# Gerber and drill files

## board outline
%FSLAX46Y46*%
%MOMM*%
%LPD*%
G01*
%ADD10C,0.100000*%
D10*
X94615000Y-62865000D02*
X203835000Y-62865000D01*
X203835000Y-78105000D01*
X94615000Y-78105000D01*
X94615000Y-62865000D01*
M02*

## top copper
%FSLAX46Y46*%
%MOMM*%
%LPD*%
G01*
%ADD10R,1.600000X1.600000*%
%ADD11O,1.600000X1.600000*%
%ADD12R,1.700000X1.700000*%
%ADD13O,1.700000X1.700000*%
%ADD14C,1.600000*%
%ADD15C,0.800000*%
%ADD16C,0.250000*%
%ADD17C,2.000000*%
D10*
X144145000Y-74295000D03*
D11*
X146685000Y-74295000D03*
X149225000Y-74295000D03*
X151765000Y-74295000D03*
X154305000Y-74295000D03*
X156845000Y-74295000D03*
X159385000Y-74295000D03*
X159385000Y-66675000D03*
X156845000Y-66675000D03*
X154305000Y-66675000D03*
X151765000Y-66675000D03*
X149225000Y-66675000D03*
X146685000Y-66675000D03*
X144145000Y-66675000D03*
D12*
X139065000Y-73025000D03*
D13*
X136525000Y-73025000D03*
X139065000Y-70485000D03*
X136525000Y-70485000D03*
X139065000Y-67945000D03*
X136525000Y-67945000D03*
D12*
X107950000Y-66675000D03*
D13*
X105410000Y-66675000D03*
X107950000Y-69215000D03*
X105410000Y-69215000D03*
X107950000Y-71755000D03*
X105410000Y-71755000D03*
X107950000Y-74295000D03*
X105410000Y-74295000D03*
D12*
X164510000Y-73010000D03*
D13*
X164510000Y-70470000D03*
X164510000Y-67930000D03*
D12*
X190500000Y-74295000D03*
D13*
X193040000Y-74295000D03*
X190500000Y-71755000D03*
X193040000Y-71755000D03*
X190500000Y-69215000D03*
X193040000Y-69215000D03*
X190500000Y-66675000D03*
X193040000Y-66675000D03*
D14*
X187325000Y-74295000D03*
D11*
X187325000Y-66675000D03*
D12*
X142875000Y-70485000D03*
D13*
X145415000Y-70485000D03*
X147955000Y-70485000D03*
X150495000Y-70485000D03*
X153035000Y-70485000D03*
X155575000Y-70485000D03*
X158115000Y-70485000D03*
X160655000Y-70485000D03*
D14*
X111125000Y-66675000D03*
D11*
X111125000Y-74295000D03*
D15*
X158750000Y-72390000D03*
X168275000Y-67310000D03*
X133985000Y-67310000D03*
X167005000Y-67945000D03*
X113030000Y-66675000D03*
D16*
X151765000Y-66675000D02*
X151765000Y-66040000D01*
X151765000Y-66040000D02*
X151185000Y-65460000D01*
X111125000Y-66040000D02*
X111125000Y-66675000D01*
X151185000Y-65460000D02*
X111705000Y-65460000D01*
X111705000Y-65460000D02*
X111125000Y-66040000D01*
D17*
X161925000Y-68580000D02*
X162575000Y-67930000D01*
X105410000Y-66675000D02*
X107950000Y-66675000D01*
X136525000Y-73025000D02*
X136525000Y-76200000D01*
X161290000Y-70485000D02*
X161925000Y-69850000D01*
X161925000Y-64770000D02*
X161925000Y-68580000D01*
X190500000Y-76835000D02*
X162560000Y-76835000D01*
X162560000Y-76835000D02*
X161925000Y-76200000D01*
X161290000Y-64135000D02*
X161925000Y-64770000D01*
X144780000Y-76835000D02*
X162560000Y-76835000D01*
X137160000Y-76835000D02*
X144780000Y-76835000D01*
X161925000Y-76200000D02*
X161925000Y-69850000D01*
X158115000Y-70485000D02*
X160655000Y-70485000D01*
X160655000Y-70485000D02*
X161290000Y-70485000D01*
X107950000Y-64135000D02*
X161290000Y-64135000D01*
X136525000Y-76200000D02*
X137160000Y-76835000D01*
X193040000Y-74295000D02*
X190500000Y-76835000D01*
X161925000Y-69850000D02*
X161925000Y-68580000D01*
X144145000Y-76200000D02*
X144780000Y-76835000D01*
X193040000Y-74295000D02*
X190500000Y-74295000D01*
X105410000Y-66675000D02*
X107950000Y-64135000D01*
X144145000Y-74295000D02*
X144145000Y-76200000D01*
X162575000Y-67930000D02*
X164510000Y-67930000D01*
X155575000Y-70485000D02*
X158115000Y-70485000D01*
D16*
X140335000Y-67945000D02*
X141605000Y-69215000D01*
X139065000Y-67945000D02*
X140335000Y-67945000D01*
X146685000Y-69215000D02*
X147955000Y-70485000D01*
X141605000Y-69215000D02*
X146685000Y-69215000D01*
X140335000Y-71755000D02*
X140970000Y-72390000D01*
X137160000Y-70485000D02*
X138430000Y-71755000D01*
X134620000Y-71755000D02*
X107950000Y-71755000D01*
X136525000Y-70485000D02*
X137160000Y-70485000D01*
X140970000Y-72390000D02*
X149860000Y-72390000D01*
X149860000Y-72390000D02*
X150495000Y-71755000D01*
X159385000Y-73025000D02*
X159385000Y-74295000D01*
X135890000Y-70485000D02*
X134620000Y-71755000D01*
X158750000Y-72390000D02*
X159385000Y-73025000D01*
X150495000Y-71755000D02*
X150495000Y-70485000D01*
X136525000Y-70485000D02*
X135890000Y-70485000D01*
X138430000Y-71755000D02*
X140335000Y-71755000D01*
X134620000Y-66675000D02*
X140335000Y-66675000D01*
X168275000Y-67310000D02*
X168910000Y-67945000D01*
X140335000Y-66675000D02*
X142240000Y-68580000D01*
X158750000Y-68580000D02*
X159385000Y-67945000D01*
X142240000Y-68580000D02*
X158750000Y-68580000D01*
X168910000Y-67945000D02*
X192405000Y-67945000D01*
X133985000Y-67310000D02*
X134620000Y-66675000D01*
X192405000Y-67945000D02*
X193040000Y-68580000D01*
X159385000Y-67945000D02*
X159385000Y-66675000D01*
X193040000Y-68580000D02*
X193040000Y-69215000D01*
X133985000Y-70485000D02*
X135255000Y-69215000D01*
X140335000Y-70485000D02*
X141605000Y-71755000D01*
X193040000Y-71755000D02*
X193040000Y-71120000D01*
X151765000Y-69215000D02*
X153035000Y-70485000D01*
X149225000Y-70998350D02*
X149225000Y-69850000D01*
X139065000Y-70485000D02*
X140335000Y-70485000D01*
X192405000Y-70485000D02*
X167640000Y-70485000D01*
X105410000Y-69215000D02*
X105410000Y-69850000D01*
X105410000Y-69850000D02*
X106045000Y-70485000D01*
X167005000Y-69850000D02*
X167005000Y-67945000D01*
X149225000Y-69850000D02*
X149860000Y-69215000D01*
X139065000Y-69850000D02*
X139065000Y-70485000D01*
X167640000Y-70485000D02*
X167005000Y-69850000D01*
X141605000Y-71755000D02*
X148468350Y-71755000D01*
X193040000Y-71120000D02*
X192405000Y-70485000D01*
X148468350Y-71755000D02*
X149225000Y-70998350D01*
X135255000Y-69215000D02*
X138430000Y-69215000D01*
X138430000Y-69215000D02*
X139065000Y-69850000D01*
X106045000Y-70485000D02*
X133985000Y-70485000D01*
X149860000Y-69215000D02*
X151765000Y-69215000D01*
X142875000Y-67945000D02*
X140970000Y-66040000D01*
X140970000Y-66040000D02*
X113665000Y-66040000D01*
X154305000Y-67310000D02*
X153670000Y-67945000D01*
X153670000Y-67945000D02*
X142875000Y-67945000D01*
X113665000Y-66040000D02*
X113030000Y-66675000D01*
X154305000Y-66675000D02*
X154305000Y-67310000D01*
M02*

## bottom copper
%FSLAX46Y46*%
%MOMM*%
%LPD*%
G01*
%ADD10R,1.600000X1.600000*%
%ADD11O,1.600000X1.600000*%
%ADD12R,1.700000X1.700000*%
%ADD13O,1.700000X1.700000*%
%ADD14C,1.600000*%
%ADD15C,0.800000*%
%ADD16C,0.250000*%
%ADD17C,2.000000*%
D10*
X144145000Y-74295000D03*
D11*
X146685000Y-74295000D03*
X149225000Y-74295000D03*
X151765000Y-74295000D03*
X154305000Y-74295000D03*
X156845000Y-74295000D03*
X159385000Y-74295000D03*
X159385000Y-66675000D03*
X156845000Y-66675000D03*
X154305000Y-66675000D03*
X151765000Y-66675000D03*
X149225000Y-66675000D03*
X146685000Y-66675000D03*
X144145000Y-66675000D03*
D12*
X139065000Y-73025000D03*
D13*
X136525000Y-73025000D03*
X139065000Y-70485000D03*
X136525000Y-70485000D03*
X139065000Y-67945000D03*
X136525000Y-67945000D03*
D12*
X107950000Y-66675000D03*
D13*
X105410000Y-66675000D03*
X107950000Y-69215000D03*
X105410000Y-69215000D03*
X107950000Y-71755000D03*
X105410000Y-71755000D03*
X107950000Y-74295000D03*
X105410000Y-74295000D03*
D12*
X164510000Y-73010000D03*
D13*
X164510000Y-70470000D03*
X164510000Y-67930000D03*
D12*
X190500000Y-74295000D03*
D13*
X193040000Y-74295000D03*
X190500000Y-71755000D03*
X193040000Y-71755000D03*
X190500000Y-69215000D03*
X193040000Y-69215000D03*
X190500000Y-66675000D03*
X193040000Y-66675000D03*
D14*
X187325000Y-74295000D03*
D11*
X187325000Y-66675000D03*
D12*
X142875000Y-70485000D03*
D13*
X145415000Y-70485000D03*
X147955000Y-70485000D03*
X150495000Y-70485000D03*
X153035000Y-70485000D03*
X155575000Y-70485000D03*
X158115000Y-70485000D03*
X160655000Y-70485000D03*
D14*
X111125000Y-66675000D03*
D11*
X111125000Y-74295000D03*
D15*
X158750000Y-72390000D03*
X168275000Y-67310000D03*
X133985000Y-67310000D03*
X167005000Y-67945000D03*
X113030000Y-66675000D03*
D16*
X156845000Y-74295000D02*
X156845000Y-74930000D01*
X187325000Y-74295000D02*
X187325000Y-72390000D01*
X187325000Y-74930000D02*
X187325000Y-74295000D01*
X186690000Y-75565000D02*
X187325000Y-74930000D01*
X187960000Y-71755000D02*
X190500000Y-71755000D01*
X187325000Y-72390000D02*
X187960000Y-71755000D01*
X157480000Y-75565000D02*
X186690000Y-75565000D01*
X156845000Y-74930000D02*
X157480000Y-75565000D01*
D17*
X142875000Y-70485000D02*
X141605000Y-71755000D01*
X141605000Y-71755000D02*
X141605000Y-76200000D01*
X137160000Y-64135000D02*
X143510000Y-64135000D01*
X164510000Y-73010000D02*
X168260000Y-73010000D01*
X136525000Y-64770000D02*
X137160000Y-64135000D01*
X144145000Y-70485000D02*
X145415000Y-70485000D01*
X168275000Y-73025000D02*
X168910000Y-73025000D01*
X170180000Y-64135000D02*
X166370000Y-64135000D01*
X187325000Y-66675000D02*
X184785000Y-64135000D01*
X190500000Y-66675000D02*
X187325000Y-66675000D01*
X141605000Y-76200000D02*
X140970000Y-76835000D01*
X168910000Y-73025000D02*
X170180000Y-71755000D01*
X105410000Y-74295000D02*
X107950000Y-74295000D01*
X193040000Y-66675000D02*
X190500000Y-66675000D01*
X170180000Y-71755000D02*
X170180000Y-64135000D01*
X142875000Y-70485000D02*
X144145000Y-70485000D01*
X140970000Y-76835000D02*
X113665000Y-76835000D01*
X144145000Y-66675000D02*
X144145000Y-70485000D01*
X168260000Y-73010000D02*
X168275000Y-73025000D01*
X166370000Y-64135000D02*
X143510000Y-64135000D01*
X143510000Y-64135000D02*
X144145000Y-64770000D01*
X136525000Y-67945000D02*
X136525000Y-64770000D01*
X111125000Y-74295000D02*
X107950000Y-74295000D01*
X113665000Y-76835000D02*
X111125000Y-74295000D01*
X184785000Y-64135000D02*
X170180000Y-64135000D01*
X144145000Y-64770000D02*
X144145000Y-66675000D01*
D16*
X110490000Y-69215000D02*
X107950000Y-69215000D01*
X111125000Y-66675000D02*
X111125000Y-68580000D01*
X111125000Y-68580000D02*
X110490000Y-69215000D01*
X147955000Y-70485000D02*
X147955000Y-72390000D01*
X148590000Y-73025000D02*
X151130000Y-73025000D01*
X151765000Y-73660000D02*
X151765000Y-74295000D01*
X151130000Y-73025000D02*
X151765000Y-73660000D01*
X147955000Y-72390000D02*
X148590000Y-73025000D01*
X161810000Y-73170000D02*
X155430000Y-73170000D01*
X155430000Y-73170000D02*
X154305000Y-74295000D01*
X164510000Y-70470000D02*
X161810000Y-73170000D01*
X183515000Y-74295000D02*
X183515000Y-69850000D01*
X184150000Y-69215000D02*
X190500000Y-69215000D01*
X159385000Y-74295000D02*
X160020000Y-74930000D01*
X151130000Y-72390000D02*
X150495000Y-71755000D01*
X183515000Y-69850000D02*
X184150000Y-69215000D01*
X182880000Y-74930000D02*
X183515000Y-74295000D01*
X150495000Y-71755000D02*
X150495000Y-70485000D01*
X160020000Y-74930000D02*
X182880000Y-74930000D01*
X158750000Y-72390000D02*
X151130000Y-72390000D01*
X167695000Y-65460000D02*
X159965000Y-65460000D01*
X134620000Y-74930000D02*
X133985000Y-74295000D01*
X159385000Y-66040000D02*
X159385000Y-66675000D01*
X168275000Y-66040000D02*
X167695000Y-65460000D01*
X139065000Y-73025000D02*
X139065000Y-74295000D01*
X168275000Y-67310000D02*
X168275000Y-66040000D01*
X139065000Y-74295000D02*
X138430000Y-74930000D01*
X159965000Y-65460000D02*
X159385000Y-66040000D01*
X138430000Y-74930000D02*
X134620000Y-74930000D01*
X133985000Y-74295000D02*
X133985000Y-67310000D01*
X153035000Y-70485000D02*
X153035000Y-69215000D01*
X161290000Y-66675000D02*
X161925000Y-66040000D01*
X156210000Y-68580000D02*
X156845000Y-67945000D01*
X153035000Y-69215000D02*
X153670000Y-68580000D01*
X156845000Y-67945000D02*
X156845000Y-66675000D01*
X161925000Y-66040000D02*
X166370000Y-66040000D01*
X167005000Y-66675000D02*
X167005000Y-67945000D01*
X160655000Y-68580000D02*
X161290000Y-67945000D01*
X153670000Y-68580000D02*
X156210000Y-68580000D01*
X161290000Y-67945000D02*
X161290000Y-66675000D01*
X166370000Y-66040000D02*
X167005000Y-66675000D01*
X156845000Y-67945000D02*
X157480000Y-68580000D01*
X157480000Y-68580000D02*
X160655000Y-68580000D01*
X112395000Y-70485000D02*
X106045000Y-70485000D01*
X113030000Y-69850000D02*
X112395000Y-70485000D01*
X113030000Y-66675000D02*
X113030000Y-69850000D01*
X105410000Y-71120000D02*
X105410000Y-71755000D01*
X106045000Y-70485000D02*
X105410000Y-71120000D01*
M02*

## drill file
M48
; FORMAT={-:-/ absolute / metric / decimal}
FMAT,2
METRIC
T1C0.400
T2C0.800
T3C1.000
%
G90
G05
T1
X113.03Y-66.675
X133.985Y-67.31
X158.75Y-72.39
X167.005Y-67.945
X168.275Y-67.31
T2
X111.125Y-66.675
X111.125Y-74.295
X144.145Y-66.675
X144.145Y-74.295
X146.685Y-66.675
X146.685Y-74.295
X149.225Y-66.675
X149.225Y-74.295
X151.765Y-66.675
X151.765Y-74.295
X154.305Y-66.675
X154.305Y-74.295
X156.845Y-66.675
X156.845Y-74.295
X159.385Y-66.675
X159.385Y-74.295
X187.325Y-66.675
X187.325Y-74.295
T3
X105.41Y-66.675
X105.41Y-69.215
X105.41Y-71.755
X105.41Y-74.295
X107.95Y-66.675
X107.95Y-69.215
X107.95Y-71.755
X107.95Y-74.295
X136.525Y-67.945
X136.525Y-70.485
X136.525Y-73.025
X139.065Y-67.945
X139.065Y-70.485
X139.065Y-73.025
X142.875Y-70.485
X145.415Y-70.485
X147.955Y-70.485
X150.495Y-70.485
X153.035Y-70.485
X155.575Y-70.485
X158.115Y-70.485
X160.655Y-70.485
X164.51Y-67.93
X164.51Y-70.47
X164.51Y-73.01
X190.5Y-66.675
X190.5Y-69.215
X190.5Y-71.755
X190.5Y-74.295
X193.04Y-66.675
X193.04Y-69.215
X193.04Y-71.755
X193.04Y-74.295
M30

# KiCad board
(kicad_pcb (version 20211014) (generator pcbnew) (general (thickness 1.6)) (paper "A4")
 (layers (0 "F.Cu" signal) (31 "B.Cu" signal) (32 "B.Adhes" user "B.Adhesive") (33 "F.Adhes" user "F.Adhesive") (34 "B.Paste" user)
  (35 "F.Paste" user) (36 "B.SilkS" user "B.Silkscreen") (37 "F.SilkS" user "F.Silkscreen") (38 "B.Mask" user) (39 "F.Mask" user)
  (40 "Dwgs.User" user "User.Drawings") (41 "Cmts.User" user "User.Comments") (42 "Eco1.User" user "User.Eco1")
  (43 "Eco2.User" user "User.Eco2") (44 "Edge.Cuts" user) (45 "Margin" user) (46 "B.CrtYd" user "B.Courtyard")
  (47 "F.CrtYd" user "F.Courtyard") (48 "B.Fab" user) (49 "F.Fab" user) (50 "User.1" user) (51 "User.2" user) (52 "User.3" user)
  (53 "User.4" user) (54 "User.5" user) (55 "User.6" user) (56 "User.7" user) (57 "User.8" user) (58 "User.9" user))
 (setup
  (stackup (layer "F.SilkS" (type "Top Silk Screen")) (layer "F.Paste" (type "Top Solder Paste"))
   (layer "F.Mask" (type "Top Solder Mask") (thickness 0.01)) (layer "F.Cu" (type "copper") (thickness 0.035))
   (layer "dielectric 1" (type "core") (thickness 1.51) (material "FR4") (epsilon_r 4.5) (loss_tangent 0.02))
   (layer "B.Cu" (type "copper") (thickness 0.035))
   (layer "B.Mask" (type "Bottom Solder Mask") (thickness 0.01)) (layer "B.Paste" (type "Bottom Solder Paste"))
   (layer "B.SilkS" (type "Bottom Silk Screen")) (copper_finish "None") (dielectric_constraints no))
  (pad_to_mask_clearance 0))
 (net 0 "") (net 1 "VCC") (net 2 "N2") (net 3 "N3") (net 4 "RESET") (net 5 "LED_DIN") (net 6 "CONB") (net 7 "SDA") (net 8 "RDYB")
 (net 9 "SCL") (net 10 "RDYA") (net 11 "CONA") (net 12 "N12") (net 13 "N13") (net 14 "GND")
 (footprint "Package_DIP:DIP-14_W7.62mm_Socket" (layer "F.Cu") (at 144.145 74.295 90)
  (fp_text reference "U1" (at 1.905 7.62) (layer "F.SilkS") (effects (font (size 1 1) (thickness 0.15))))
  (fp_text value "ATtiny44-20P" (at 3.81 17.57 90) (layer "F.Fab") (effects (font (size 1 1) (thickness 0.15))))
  (pad "1" thru_hole rect (at 0 0 90) (size 1.6 1.6) (drill 0.8) (layers *.Cu *.Mask) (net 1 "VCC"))
  (pad "2" thru_hole oval (at 0 2.54 90) (size 1.6 1.6) (drill 0.8) (layers *.Cu *.Mask) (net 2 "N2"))
  (pad "3" thru_hole oval (at 0 5.08 90) (size 1.6 1.6) (drill 0.8) (layers *.Cu *.Mask) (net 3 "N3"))
  (pad "4" thru_hole oval (at 0 7.62 90) (size 1.6 1.6) (drill 0.8) (layers *.Cu *.Mask) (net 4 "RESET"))
  (pad "5" thru_hole oval (at 0 10.16 90) (size 1.6 1.6) (drill 0.8) (layers *.Cu *.Mask) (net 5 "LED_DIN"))
  (pad "6" thru_hole oval (at 0 12.7 90) (size 1.6 1.6) (drill 0.8) (layers *.Cu *.Mask) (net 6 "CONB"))
  (pad "7" thru_hole oval (at 0 15.24 90) (size 1.6 1.6) (drill 0.8) (layers *.Cu *.Mask) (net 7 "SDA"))
  (pad "8" thru_hole oval (at 7.62 15.24 90) (size 1.6 1.6) (drill 0.8) (layers *.Cu *.Mask) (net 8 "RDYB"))
  (pad "9" thru_hole oval (at 7.62 12.7 90) (size 1.6 1.6) (drill 0.8) (layers *.Cu *.Mask) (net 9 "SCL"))
  (pad "10" thru_hole oval (at 7.62 10.16 90) (size 1.6 1.6) (drill 0.8) (layers *.Cu *.Mask) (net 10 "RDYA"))
  (pad "11" thru_hole oval (at 7.62 7.62 90) (size 1.6 1.6) (drill 0.8) (layers *.Cu *.Mask) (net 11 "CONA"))
  (pad "12" thru_hole oval (at 7.62 5.08 90) (size 1.6 1.6) (drill 0.8) (layers *.Cu *.Mask) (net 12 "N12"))
  (pad "13" thru_hole oval (at 7.62 2.54 90) (size 1.6 1.6) (drill 0.8) (layers *.Cu *.Mask) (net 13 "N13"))
  (pad "14" thru_hole oval (at 7.62 0 90) (size 1.6 1.6) (drill 0.8) (layers *.Cu *.Mask) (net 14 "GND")))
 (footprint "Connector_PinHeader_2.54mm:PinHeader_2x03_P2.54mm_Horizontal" (layer "F.Cu") (at 139.065 73.025 180)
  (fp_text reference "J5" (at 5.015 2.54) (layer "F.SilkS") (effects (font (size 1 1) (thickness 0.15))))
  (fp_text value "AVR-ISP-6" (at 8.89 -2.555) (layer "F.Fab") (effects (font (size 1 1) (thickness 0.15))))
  (pad "1" thru_hole rect (at 0 0 180) (size 1.7 1.7) (drill 1) (layers *.Cu *.Mask) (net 8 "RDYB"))
  (pad "2" thru_hole oval (at 2.54 0 180) (size 1.7 1.7) (drill 1) (layers *.Cu *.Mask) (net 1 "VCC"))
  (pad "3" thru_hole oval (at 0 2.54 180) (size 1.7 1.7) (drill 1) (layers *.Cu *.Mask) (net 9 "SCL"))
  (pad "4" thru_hole oval (at 2.54 2.54 180) (size 1.7 1.7) (drill 1) (layers *.Cu *.Mask) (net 7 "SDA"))
  (pad "5" thru_hole oval (at 0 5.08 180) (size 1.7 1.7) (drill 1) (layers *.Cu *.Mask) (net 4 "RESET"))
  (pad "6" thru_hole oval (at 2.54 5.08 180) (size 1.7 1.7) (drill 1) (layers *.Cu *.Mask) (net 14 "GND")))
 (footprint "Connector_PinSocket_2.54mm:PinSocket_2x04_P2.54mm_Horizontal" (layer "F.Cu") (at 107.95 66.675)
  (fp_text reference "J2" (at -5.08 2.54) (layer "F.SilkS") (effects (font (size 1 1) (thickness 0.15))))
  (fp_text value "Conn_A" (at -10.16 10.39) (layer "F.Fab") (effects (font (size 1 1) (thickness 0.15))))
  (pad "1" thru_hole rect (at 0 0) (size 1.7 1.7) (drill 1) (layers *.Cu *.Mask) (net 1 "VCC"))
  (pad "2" thru_hole oval (at -2.54 0) (size 1.7 1.7) (drill 1) (layers *.Cu *.Mask) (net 1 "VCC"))
  (pad "3" thru_hole oval (at 0 2.54) (size 1.7 1.7) (drill 1) (layers *.Cu *.Mask) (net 11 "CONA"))
  (pad "4" thru_hole oval (at -2.54 2.54) (size 1.7 1.7) (drill 1) (layers *.Cu *.Mask) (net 9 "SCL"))
  (pad "5" thru_hole oval (at 0 5.08) (size 1.7 1.7) (drill 1) (layers *.Cu *.Mask) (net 7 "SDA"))
  (pad "6" thru_hole oval (at -2.54 5.08) (size 1.7 1.7) (drill 1) (layers *.Cu *.Mask) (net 10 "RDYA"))
  (pad "7" thru_hole oval (at 0 7.62) (size 1.7 1.7) (drill 1) (layers *.Cu *.Mask) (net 14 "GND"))
  (pad "8" thru_hole oval (at -2.54 7.62) (size 1.7 1.7) (drill 1) (layers *.Cu *.Mask) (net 14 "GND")))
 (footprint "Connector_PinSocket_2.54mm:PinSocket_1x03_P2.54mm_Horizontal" (layer "F.Cu") (at 164.51 73.01 180)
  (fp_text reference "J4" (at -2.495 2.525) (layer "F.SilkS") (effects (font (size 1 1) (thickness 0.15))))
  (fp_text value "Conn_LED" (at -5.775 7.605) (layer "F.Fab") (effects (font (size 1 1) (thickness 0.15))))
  (pad "1" thru_hole rect (at 0 0 180) (size 1.7 1.7) (drill 1) (layers *.Cu *.Mask) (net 14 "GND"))
  (pad "2" thru_hole oval (at 0 2.54 180) (size 1.7 1.7) (drill 1) (layers *.Cu *.Mask) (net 5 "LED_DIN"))
  (pad "3" thru_hole oval (at 0 5.08 180) (size 1.7 1.7) (drill 1) (layers *.Cu *.Mask) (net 1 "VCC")))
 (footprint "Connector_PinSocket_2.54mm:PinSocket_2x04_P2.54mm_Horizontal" (layer "F.Cu") (at 190.5 74.295 180)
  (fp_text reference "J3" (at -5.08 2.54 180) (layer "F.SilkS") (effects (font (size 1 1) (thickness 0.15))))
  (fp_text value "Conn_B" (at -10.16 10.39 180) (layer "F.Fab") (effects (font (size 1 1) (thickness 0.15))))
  (pad "1" thru_hole rect (at 0 0 180) (size 1.7 1.7) (drill 1) (layers *.Cu *.Mask) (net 1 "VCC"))
  (pad "2" thru_hole oval (at -2.54 0 180) (size 1.7 1.7) (drill 1) (layers *.Cu *.Mask) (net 1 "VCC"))
  (pad "3" thru_hole oval (at 0 2.54 180) (size 1.7 1.7) (drill 1) (layers *.Cu *.Mask) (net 6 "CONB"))
  (pad "4" thru_hole oval (at -2.54 2.54 180) (size 1.7 1.7) (drill 1) (layers *.Cu *.Mask) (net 9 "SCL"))
  (pad "5" thru_hole oval (at 0 5.08 180) (size 1.7 1.7) (drill 1) (layers *.Cu *.Mask) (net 7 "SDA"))
  (pad "6" thru_hole oval (at -2.54 5.08 180) (size 1.7 1.7) (drill 1) (layers *.Cu *.Mask) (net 8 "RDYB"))
  (pad "7" thru_hole oval (at 0 7.62 180) (size 1.7 1.7) (drill 1) (layers *.Cu *.Mask) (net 14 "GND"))
  (pad "8" thru_hole oval (at -2.54 7.62 180) (size 1.7 1.7) (drill 1) (layers *.Cu *.Mask) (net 14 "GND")))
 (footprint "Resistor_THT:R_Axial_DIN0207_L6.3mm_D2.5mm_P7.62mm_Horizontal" (layer "B.Cu") (at 187.325 74.295 90)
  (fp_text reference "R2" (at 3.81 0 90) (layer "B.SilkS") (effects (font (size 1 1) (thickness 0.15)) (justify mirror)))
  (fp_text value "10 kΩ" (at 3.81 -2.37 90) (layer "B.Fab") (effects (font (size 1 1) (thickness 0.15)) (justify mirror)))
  (pad "1" thru_hole circle (at 0 0 90) (size 1.6 1.6) (drill 0.8) (layers *.Cu *.Mask) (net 6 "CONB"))
  (pad "2" thru_hole oval (at 7.62 0 90) (size 1.6 1.6) (drill 0.8) (layers *.Cu *.Mask) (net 14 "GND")))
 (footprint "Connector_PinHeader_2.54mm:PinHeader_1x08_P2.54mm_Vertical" (layer "B.Cu") (at 142.875 70.485 -90)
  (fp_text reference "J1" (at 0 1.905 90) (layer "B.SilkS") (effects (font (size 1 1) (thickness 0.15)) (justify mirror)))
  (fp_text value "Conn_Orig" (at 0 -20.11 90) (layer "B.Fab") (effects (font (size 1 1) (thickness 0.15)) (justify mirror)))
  (pad "1" thru_hole rect (at 0 0 270) (size 1.7 1.7) (drill 1) (layers *.Cu *.Mask) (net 14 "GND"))
  (pad "2" thru_hole oval (at 0 -2.54 270) (size 1.7 1.7) (drill 1) (layers *.Cu *.Mask) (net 14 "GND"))
  (pad "3" thru_hole oval (at 0 -5.08 270) (size 1.7 1.7) (drill 1) (layers *.Cu *.Mask) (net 4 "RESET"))
  (pad "4" thru_hole oval (at 0 -7.62 270) (size 1.7 1.7) (drill 1) (layers *.Cu *.Mask) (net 7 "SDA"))
  (pad "5" thru_hole oval (at 0 -10.16 270) (size 1.7 1.7) (drill 1) (layers *.Cu *.Mask) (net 9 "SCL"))
  (pad "6" thru_hole oval (at 0 -12.7 270) (size 1.7 1.7) (drill 1) (layers *.Cu *.Mask) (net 1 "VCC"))
  (pad "7" thru_hole oval (at 0 -15.24 270) (size 1.7 1.7) (drill 1) (layers *.Cu *.Mask) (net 1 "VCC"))
  (pad "8" thru_hole oval (at 0 -17.78 270) (size 1.7 1.7) (drill 1) (layers *.Cu *.Mask) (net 1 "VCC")))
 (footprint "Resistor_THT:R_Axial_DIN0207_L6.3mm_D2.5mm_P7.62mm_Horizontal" (layer "B.Cu") (at 111.125 66.675 -90)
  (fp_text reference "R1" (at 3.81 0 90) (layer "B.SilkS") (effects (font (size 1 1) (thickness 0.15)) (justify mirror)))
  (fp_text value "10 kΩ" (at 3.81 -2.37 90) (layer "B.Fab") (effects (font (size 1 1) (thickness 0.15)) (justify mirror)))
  (pad "1" thru_hole circle (at 0 0 270) (size 1.6 1.6) (drill 0.8) (layers *.Cu *.Mask) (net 11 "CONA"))
  (pad "2" thru_hole oval (at 7.62 0 270) (size 1.6 1.6) (drill 0.8) (layers *.Cu *.Mask) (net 14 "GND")))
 (gr_rect (start 94.615 62.865) (end 203.835 78.105) (layer "Edge.Cuts") (width 0.1) (fill none))
 (segment (start 156.845 74.295) (end 156.845 74.93) (width 0.25) (layer "B.Cu") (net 6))
 (segment (start 187.325 74.295) (end 187.325 72.39) (width 0.25) (layer "B.Cu") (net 6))
 (segment (start 187.325 74.93) (end 187.325 74.295) (width 0.25) (layer "B.Cu") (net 6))
 (segment (start 186.69 75.565) (end 187.325 74.93) (width 0.25) (layer "B.Cu") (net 6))
 (segment (start 187.96 71.755) (end 190.5 71.755) (width 0.25) (layer "B.Cu") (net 6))
 (segment (start 187.325 72.39) (end 187.96 71.755) (width 0.25) (layer "B.Cu") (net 6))
 (segment (start 157.48 75.565) (end 186.69 75.565) (width 0.25) (layer "B.Cu") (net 6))
 (segment (start 156.845 74.93) (end 157.48 75.565) (width 0.25) (layer "B.Cu") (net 6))
 (segment (start 142.875 70.485) (end 141.605 71.755) (width 2) (layer "B.Cu") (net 14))
 (segment (start 141.605 71.755) (end 141.605 76.2) (width 2) (layer "B.Cu") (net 14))
 (segment (start 137.16 64.135) (end 143.51 64.135) (width 2) (layer "B.Cu") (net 14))
 (segment (start 164.51 73.01) (end 168.26 73.01) (width 2) (layer "B.Cu") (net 14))
 (segment (start 136.525 64.77) (end 137.16 64.135) (width 2) (layer "B.Cu") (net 14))
 (segment (start 144.145 70.485) (end 145.415 70.485) (width 2) (layer "B.Cu") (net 14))
 (segment (start 168.275 73.025) (end 168.91 73.025) (width 2) (layer "B.Cu") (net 14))
 (segment (start 170.18 64.135) (end 166.37 64.135) (width 2) (layer "B.Cu") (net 14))
 (segment (start 187.325 66.675) (end 184.785 64.135) (width 2) (layer "B.Cu") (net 14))
 (segment (start 190.5 66.675) (end 187.325 66.675) (width 2) (layer "B.Cu") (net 14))
 (segment (start 141.605 76.2) (end 140.97 76.835) (width 2) (layer "B.Cu") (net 14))
 (segment (start 168.91 73.025) (end 170.18 71.755) (width 2) (layer "B.Cu") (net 14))
 (segment (start 105.41 74.295) (end 107.95 74.295) (width 2) (layer "B.Cu") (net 14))
 (segment (start 193.04 66.675) (end 190.5 66.675) (width 2) (layer "B.Cu") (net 14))
 (segment (start 170.18 71.755) (end 170.18 64.135) (width 2) (layer "B.Cu") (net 14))
 (segment (start 142.875 70.485) (end 144.145 70.485) (width 2) (layer "B.Cu") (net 14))
 (segment (start 140.97 76.835) (end 113.665 76.835) (width 2) (layer "B.Cu") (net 14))
 (segment (start 144.145 66.675) (end 144.145 70.485) (width 2) (layer "B.Cu") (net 14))
 (segment (start 168.26 73.01) (end 168.275 73.025) (width 2) (layer "B.Cu") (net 14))
 (segment (start 166.37 64.135) (end 143.51 64.135) (width 2) (layer "B.Cu") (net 14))
 (segment (start 143.51 64.135) (end 144.145 64.77) (width 2) (layer "B.Cu") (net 14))
 (segment (start 136.525 67.945) (end 136.525 64.77) (width 2) (layer "B.Cu") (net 14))
 (segment (start 111.125 74.295) (end 107.95 74.295) (width 2) (layer "B.Cu") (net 14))
 (segment (start 113.665 76.835) (end 111.125 74.295) (width 2) (layer "B.Cu") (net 14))
 (segment (start 184.785 64.135) (end 170.18 64.135) (width 2) (layer "B.Cu") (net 14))
 (segment (start 144.145 64.77) (end 144.145 66.675) (width 2) (layer "B.Cu") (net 14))
 (segment (start 151.765 66.675) (end 151.765 66.04) (width 0.25) (layer "F.Cu") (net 11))
 (segment (start 151.765 66.04) (end 151.185 65.46) (width 0.25) (layer "F.Cu") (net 11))
 (segment (start 111.125 66.04) (end 111.125 66.675) (width 0.25) (layer "F.Cu") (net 11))
 (segment (start 151.185 65.46) (end 111.705 65.46) (width 0.25) (layer "F.Cu") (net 11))
 (segment (start 111.705 65.46) (end 111.125 66.04) (width 0.25) (layer "F.Cu") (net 11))
 (segment (start 110.49 69.215) (end 107.95 69.215) (width 0.25) (layer "B.Cu") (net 11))
 (segment (start 111.125 66.675) (end 111.125 68.58) (width 0.25) (layer "B.Cu") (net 11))
 (segment (start 111.125 68.58) (end 110.49 69.215) (width 0.25) (layer "B.Cu") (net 11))
 (segment (start 161.925 68.58) (end 162.575 67.93) (width 2) (layer "F.Cu") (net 1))
 (segment (start 105.41 66.675) (end 107.95 66.675) (width 2) (layer "F.Cu") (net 1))
 (segment (start 136.525 73.025) (end 136.525 76.2) (width 2) (layer "F.Cu") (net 1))
 (segment (start 161.29 70.485) (end 161.925 69.85) (width 2) (layer "F.Cu") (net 1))
 (segment (start 161.925 64.77) (end 161.925 68.58) (width 2) (layer "F.Cu") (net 1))
 (segment (start 190.5 76.835) (end 162.56 76.835) (width 2) (layer "F.Cu") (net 1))
 (segment (start 162.56 76.835) (end 161.925 76.2) (width 2) (layer "F.Cu") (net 1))
 (segment (start 161.29 64.135) (end 161.925 64.77) (width 2) (layer "F.Cu") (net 1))
 (segment (start 144.78 76.835) (end 162.56 76.835) (width 2) (layer "F.Cu") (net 1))
 (segment (start 137.16 76.835) (end 144.78 76.835) (width 2) (layer "F.Cu") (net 1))
 (segment (start 161.925 76.2) (end 161.925 69.85) (width 2) (layer "F.Cu") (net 1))
 (segment (start 158.115 70.485) (end 160.655 70.485) (width 2) (layer "F.Cu") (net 1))
 (segment (start 160.655 70.485) (end 161.29 70.485) (width 2) (layer "F.Cu") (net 1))
 (segment (start 107.95 64.135) (end 161.29 64.135) (width 2) (layer "F.Cu") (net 1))
 (segment (start 136.525 76.2) (end 137.16 76.835) (width 2) (layer "F.Cu") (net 1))
 (segment (start 193.04 74.295) (end 190.5 76.835) (width 2) (layer "F.Cu") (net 1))
 (segment (start 161.925 69.85) (end 161.925 68.58) (width 2) (layer "F.Cu") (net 1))
 (segment (start 144.145 76.2) (end 144.78 76.835) (width 2) (layer "F.Cu") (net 1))
 (segment (start 193.04 74.295) (end 190.5 74.295) (width 2) (layer "F.Cu") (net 1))
 (segment (start 105.41 66.675) (end 107.95 64.135) (width 2) (layer "F.Cu") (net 1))
 (segment (start 144.145 74.295) (end 144.145 76.2) (width 2) (layer "F.Cu") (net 1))
 (segment (start 162.575 67.93) (end 164.51 67.93) (width 2) (layer "F.Cu") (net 1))
 (segment (start 155.575 70.485) (end 158.115 70.485) (width 2) (layer "F.Cu") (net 1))
 (segment (start 140.335 67.945) (end 141.605 69.215) (width 0.25) (layer "F.Cu") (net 4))
 (segment (start 139.065 67.945) (end 140.335 67.945) (width 0.25) (layer "F.Cu") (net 4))
 (segment (start 146.685 69.215) (end 147.955 70.485) (width 0.25) (layer "F.Cu") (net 4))
 (segment (start 141.605 69.215) (end 146.685 69.215) (width 0.25) (layer "F.Cu") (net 4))
 (segment (start 147.955 70.485) (end 147.955 72.39) (width 0.25) (layer "B.Cu") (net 4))
 (segment (start 148.59 73.025) (end 151.13 73.025) (width 0.25) (layer "B.Cu") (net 4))
 (segment (start 151.765 73.66) (end 151.765 74.295) (width 0.25) (layer "B.Cu") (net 4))
 (segment (start 151.13 73.025) (end 151.765 73.66) (width 0.25) (layer "B.Cu") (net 4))
 (segment (start 147.955 72.39) (end 148.59 73.025) (width 0.25) (layer "B.Cu") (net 4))
 (segment (start 161.81 73.17) (end 155.43 73.17) (width 0.25) (layer "B.Cu") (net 5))
 (segment (start 155.43 73.17) (end 154.305 74.295) (width 0.25) (layer "B.Cu") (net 5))
 (segment (start 164.51 70.47) (end 161.81 73.17) (width 0.25) (layer "B.Cu") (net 5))
 (segment (start 140.335 71.755) (end 140.97 72.39) (width 0.25) (layer "F.Cu") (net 7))
 (segment (start 137.16 70.485) (end 138.43 71.755) (width 0.25) (layer "F.Cu") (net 7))
 (segment (start 134.62 71.755) (end 107.95 71.755) (width 0.25) (layer "F.Cu") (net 7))
 (segment (start 136.525 70.485) (end 137.16 70.485) (width 0.25) (layer "F.Cu") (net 7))
 (segment (start 140.97 72.39) (end 149.86 72.39) (width 0.25) (layer "F.Cu") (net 7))
 (segment (start 149.86 72.39) (end 150.495 71.755) (width 0.25) (layer "F.Cu") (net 7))
 (segment (start 159.385 73.025) (end 159.385 74.295) (width 0.25) (layer "F.Cu") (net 7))
 (segment (start 135.89 70.485) (end 134.62 71.755) (width 0.25) (layer "F.Cu") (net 7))
 (segment (start 158.75 72.39) (end 159.385 73.025) (width 0.25) (layer "F.Cu") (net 7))
 (segment (start 150.495 71.755) (end 150.495 70.485) (width 0.25) (layer "F.Cu") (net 7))
 (segment (start 136.525 70.485) (end 135.89 70.485) (width 0.25) (layer "F.Cu") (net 7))
 (segment (start 138.43 71.755) (end 140.335 71.755) (width 0.25) (layer "F.Cu") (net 7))
 (via (at 158.75 72.39) (size 0.8) (drill 0.4) (layers "F.Cu" "B.Cu") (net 7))
 (segment (start 183.515 74.295) (end 183.515 69.85) (width 0.25) (layer "B.Cu") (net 7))
 (segment (start 184.15 69.215) (end 190.5 69.215) (width 0.25) (layer "B.Cu") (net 7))
 (segment (start 159.385 74.295) (end 160.02 74.93) (width 0.25) (layer "B.Cu") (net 7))
 (segment (start 151.13 72.39) (end 150.495 71.755) (width 0.25) (layer "B.Cu") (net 7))
 (segment (start 183.515 69.85) (end 184.15 69.215) (width 0.25) (layer "B.Cu") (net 7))
 (segment (start 182.88 74.93) (end 183.515 74.295) (width 0.25) (layer "B.Cu") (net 7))
 (segment (start 150.495 71.755) (end 150.495 70.485) (width 0.25) (layer "B.Cu") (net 7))
 (segment (start 160.02 74.93) (end 182.88 74.93) (width 0.25) (layer "B.Cu") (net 7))
 (segment (start 158.75 72.39) (end 151.13 72.39) (width 0.25) (layer "B.Cu") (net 7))
 (segment (start 134.62 66.675) (end 140.335 66.675) (width 0.25) (layer "F.Cu") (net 8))
 (segment (start 168.275 67.31) (end 168.91 67.945) (width 0.25) (layer "F.Cu") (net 8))
 (segment (start 140.335 66.675) (end 142.24 68.58) (width 0.25) (layer "F.Cu") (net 8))
 (segment (start 158.75 68.58) (end 159.385 67.945) (width 0.25) (layer "F.Cu") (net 8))
 (segment (start 142.24 68.58) (end 158.75 68.58) (width 0.25) (layer "F.Cu") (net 8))
 (segment (start 168.91 67.945) (end 192.405 67.945) (width 0.25) (layer "F.Cu") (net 8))
 (segment (start 133.985 67.31) (end 134.62 66.675) (width 0.25) (layer "F.Cu") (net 8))
 (segment (start 192.405 67.945) (end 193.04 68.58) (width 0.25) (layer "F.Cu") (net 8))
 (segment (start 159.385 67.945) (end 159.385 66.675) (width 0.25) (layer "F.Cu") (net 8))
 (segment (start 193.04 68.58) (end 193.04 69.215) (width 0.25) (layer "F.Cu") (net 8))
 (via (at 168.275 67.31) (size 0.8) (drill 0.4) (layers "F.Cu" "B.Cu") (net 8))
 (via (at 133.985 67.31) (size 0.8) (drill 0.4) (layers "F.Cu" "B.Cu") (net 8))
 (segment (start 167.695 65.46) (end 159.965 65.46) (width 0.25) (layer "B.Cu") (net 8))
 (segment (start 134.62 74.93) (end 133.985 74.295) (width 0.25) (layer "B.Cu") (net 8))
 (segment (start 159.385 66.04) (end 159.385 66.675) (width 0.25) (layer "B.Cu") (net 8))
 (segment (start 168.275 66.04) (end 167.695 65.46) (width 0.25) (layer "B.Cu") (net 8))
 (segment (start 139.065 73.025) (end 139.065 74.295) (width 0.25) (layer "B.Cu") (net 8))
 (segment (start 168.275 67.31) (end 168.275 66.04) (width 0.25) (layer "B.Cu") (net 8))
 (segment (start 139.065 74.295) (end 138.43 74.93) (width 0.25) (layer "B.Cu") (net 8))
 (segment (start 159.965 65.46) (end 159.385 66.04) (width 0.25) (layer "B.Cu") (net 8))
 (segment (start 138.43 74.93) (end 134.62 74.93) (width 0.25) (layer "B.Cu") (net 8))
 (segment (start 133.985 74.295) (end 133.985 67.31) (width 0.25) (layer "B.Cu") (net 8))
 (segment (start 133.985 70.485) (end 135.255 69.215) (width 0.25) (layer "F.Cu") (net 9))
 (segment (start 140.335 70.485) (end 141.605 71.755) (width 0.25) (layer "F.Cu") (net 9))
 (segment (start 193.04 71.755) (end 193.04 71.12) (width 0.25) (layer "F.Cu") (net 9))
 (segment (start 151.765 69.215) (end 153.035 70.485) (width 0.25) (layer "F.Cu") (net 9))
 (segment (start 149.225 70.99835) (end 149.225 69.85) (width 0.25) (layer "F.Cu") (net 9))
 (segment (start 139.065 70.485) (end 140.335 70.485) (width 0.25) (layer "F.Cu") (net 9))
 (segment (start 192.405 70.485) (end 167.64 70.485) (width 0.25) (layer "F.Cu") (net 9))
 (segment (start 105.41 69.215) (end 105.41 69.85) (width 0.25) (layer "F.Cu") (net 9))
 (segment (start 105.41 69.85) (end 106.045 70.485) (width 0.25) (layer "F.Cu") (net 9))
 (segment (start 167.005 69.85) (end 167.005 67.945) (width 0.25) (layer "F.Cu") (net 9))
 (segment (start 149.225 69.85) (end 149.86 69.215) (width 0.25) (layer "F.Cu") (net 9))
 (segment (start 139.065 69.85) (end 139.065 70.485) (width 0.25) (layer "F.Cu") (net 9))
 (segment (start 167.64 70.485) (end 167.005 69.85) (width 0.25) (layer "F.Cu") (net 9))
 (segment (start 141.605 71.755) (end 148.46835 71.755) (width 0.25) (layer "F.Cu") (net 9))
 (segment (start 193.04 71.12) (end 192.405 70.485) (width 0.25) (layer "F.Cu") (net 9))
 (segment (start 148.46835 71.755) (end 149.225 70.99835) (width 0.25) (layer "F.Cu") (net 9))
 (segment (start 135.255 69.215) (end 138.43 69.215) (width 0.25) (layer "F.Cu") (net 9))
 (segment (start 138.43 69.215) (end 139.065 69.85) (width 0.25) (layer "F.Cu") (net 9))
 (segment (start 106.045 70.485) (end 133.985 70.485) (width 0.25) (layer "F.Cu") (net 9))
 (segment (start 149.86 69.215) (end 151.765 69.215) (width 0.25) (layer "F.Cu") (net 9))
 (via (at 167.005 67.945) (size 0.8) (drill 0.4) (layers "F.Cu" "B.Cu") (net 9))
 (segment (start 153.035 70.485) (end 153.035 69.215) (width 0.25) (layer "B.Cu") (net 9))
 (segment (start 161.29 66.675) (end 161.925 66.04) (width 0.25) (layer "B.Cu") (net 9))
 (segment (start 156.21 68.58) (end 156.845 67.945) (width 0.25) (layer "B.Cu") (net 9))
 (segment (start 153.035 69.215) (end 153.67 68.58) (width 0.25) (layer "B.Cu") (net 9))
 (segment (start 156.845 67.945) (end 156.845 66.675) (width 0.25) (layer "B.Cu") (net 9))
 (segment (start 161.925 66.04) (end 166.37 66.04) (width 0.25) (layer "B.Cu") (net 9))
 (segment (start 167.005 66.675) (end 167.005 67.945) (width 0.25) (layer "B.Cu") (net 9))
 (segment (start 160.655 68.58) (end 161.29 67.945) (width 0.25) (layer "B.Cu") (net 9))
 (segment (start 153.67 68.58) (end 156.21 68.58) (width 0.25) (layer "B.Cu") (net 9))
 (segment (start 161.29 67.945) (end 161.29 66.675) (width 0.25) (layer "B.Cu") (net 9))
 (segment (start 166.37 66.04) (end 167.005 66.675) (width 0.25) (layer "B.Cu") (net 9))
 (segment (start 156.845 67.945) (end 157.48 68.58) (width 0.25) (layer "B.Cu") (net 9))
 (segment (start 157.48 68.58) (end 160.655 68.58) (width 0.25) (layer "B.Cu") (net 9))
 (segment (start 142.875 67.945) (end 140.97 66.04) (width 0.25) (layer "F.Cu") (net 10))
 (segment (start 140.97 66.04) (end 113.665 66.04) (width 0.25) (layer "F.Cu") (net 10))
 (segment (start 154.305 67.31) (end 153.67 67.945) (width 0.25) (layer "F.Cu") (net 10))
 (segment (start 153.67 67.945) (end 142.875 67.945) (width 0.25) (layer "F.Cu") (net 10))
 (segment (start 113.665 66.04) (end 113.03 66.675) (width 0.25) (layer "F.Cu") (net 10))
 (segment (start 154.305 66.675) (end 154.305 67.31) (width 0.25) (layer "F.Cu") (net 10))
 (via (at 113.03 66.675) (size 0.8) (drill 0.4) (layers "F.Cu" "B.Cu") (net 10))
 (segment (start 112.395 70.485) (end 106.045 70.485) (width 0.25) (layer "B.Cu") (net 10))
 (segment (start 113.03 69.85) (end 112.395 70.485) (width 0.25) (layer "B.Cu") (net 10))
 (segment (start 113.03 66.675) (end 113.03 69.85) (width 0.25) (layer "B.Cu") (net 10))
 (segment (start 105.41 71.12) (end 105.41 71.755) (width 0.25) (layer "B.Cu") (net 10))
 (segment (start 106.045 70.485) (end 105.41 71.12) (width 0.25) (layer "B.Cu") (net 10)))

